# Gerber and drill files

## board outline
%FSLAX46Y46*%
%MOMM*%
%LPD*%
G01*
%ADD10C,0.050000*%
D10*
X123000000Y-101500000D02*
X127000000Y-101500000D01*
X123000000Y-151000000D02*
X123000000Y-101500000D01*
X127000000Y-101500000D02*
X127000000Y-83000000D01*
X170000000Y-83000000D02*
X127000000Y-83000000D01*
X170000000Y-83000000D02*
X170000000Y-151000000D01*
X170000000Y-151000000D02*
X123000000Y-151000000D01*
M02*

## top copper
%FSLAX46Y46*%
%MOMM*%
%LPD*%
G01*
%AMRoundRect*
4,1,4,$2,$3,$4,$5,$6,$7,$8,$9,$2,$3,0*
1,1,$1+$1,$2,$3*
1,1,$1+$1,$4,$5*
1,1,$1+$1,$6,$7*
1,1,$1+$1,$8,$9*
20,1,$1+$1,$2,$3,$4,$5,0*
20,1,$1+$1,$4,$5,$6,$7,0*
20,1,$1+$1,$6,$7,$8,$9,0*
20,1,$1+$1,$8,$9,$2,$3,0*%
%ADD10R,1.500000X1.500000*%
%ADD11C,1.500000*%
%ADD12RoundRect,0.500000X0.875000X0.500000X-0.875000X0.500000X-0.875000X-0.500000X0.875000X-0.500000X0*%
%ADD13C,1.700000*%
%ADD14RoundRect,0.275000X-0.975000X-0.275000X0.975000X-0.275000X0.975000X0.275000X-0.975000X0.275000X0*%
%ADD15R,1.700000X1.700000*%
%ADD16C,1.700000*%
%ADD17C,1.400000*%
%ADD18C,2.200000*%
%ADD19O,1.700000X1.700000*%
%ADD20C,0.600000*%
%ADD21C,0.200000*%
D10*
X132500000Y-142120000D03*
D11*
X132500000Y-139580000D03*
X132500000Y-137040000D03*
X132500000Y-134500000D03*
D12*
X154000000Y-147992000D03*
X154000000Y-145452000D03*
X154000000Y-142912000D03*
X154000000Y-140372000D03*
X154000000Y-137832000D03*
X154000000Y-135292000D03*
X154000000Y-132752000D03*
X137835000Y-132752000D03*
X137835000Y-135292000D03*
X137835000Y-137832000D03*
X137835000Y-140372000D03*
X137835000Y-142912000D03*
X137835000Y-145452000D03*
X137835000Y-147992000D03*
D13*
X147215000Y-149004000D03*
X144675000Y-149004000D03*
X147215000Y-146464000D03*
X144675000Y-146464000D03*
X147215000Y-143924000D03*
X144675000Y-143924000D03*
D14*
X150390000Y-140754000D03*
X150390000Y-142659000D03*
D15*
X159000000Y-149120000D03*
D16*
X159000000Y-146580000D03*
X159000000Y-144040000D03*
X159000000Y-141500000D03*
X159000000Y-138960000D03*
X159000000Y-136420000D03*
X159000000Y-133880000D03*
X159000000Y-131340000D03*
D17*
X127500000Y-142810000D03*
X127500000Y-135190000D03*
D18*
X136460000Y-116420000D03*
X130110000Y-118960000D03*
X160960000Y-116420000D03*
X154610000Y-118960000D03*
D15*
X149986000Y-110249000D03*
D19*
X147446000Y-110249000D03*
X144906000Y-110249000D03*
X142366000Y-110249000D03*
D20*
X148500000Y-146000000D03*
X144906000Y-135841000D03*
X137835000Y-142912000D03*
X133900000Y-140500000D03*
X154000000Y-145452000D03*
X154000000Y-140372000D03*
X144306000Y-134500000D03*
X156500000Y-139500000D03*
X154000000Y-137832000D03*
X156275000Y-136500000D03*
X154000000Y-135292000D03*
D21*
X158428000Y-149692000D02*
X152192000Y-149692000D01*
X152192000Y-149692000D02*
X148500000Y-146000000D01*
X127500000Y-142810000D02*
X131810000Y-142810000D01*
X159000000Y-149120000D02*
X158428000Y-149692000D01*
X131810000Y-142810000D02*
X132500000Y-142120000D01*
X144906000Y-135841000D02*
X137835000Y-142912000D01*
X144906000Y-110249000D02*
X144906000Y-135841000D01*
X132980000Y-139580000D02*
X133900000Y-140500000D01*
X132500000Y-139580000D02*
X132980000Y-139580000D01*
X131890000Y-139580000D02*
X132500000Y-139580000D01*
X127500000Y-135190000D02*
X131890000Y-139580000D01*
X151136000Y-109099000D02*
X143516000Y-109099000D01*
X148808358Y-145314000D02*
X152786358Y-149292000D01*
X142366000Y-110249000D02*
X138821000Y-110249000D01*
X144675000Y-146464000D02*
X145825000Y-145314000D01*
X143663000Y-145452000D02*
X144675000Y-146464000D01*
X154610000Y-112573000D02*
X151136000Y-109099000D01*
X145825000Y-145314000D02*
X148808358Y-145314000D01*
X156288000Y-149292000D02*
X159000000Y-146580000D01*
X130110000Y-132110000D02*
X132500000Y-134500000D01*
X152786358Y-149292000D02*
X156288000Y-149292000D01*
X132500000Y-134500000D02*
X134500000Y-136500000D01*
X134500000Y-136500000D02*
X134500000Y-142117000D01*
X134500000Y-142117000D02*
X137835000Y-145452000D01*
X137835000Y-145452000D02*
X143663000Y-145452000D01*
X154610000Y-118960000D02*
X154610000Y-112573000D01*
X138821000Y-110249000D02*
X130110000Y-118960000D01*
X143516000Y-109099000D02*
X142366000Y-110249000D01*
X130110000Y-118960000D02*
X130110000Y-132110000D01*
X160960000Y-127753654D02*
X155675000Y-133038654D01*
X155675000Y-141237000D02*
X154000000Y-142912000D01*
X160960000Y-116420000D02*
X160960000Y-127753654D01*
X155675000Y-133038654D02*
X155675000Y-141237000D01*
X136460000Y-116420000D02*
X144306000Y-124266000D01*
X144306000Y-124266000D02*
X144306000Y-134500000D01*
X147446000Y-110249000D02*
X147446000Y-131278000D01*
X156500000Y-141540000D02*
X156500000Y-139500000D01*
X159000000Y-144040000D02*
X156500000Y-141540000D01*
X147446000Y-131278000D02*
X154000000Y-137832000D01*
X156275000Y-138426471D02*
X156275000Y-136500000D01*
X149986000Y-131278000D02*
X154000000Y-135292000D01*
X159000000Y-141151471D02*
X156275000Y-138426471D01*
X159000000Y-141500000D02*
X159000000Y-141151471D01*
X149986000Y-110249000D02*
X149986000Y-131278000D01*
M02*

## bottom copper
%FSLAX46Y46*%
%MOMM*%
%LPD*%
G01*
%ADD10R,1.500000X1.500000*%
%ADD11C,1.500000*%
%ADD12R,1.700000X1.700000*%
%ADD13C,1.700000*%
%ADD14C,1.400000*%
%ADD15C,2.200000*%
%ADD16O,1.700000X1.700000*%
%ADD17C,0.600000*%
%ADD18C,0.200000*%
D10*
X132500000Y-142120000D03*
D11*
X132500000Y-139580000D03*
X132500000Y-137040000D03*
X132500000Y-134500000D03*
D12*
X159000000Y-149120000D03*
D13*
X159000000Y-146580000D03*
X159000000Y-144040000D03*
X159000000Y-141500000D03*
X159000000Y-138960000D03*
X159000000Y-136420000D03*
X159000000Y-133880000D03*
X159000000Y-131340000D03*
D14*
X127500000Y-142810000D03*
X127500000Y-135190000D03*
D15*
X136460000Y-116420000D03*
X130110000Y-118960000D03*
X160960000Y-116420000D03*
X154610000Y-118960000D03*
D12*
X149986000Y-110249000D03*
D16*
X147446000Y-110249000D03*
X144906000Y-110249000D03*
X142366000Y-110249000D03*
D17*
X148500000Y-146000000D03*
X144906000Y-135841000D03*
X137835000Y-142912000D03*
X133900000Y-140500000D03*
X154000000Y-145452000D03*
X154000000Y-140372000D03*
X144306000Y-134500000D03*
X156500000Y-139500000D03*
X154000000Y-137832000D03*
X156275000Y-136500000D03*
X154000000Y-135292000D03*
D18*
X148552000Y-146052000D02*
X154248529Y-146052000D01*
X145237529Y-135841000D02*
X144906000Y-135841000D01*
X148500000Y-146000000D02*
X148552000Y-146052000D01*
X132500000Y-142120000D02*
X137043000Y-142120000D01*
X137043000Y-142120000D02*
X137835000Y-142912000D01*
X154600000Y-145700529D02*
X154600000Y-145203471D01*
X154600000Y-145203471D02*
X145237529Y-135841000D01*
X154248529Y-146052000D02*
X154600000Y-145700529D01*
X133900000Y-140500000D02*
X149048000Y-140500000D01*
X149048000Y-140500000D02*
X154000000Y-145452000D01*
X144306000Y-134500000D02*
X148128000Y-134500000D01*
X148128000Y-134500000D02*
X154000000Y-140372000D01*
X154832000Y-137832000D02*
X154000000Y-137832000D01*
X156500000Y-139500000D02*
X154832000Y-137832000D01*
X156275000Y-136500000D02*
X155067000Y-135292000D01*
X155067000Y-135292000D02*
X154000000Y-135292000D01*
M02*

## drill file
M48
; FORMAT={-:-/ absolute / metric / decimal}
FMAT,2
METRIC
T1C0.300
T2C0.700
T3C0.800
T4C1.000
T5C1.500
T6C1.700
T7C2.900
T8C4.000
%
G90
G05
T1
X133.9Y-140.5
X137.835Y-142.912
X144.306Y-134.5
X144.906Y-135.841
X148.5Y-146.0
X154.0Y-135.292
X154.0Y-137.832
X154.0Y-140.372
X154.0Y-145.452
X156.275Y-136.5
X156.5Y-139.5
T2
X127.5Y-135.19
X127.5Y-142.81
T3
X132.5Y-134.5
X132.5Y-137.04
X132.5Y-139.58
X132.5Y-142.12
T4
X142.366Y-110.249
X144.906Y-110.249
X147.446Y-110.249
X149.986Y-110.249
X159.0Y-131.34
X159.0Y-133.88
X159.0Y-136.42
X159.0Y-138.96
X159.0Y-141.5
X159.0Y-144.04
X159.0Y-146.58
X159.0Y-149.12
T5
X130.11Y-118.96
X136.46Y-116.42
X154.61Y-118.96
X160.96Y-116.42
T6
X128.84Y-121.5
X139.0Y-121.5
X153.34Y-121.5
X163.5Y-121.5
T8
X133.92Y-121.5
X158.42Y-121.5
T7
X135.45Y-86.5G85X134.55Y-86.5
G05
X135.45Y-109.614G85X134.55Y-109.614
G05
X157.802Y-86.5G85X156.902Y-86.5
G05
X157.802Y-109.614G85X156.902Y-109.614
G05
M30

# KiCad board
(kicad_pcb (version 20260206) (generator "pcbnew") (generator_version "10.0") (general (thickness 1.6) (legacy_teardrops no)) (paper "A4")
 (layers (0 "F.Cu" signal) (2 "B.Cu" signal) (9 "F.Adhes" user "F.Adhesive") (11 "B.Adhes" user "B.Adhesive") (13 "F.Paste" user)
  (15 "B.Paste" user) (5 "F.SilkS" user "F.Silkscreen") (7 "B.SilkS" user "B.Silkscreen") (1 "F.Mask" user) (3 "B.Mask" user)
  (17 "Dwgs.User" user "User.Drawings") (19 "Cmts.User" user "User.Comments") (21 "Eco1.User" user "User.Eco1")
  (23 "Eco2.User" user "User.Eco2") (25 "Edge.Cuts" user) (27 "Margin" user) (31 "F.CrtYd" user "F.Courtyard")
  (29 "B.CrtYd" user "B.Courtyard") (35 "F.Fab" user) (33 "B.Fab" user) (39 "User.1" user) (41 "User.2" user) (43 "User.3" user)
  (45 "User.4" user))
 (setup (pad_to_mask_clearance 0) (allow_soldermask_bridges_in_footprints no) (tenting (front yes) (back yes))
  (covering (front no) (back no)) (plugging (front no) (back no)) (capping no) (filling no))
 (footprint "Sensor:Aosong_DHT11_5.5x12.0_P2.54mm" (layer "F.Cu") (at 132.5 142.12 180)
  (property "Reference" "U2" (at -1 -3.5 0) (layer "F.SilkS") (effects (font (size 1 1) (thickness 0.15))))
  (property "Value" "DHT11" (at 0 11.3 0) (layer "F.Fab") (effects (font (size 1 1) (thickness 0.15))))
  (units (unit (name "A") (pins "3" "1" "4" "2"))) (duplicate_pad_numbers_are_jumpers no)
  (pad "1" thru_hole rect (at 0 0 180) (size 1.5 1.5) (drill 0.8) (layers "*.Cu" "*.Mask") (remove_unused_layers no) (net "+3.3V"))
  (pad "2" thru_hole circle (at 0 2.54 180) (size 1.5 1.5) (drill 0.8) (layers "*.Cu" "*.Mask") (remove_unused_layers no)
   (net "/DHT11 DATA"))
  (pad "3" thru_hole circle (at 0 5.08 180) (size 1.5 1.5) (drill 0.8) (layers "*.Cu" "*.Mask") (remove_unused_layers no)
   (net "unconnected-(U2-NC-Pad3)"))
  (pad "4" thru_hole circle (at 0 7.62 180) (size 1.5 1.5) (drill 0.8) (layers "*.Cu" "*.Mask") (remove_unused_layers no) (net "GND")))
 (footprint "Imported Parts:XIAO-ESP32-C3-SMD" (layer "F.Cu") (at 154.835 129.872 180)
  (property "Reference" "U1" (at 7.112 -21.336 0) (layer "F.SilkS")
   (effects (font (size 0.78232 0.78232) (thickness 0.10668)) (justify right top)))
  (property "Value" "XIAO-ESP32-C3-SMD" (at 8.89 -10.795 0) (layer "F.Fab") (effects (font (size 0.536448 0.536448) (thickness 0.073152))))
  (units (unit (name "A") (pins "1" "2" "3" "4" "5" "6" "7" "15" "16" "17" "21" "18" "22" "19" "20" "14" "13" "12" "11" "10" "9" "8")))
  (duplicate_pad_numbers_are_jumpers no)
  (pad "1" smd roundrect (at 0.835 -18.12 180) (size 2.75 2) (layers "F.Cu" "F.Mask" "F.Paste") (roundrect_rratio 0.25)
   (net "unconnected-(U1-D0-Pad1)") (solder_mask_margin 0.0508) (thermal_bridge_angle 45))
  (pad "2" smd roundrect (at 0.835 -15.58 180) (size 2.75 2) (layers "F.Cu" "F.Mask" "F.Paste") (roundrect_rratio 0.25) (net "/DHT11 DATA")
   (solder_mask_margin 0.0508) (thermal_bridge_angle 45))
  (pad "3" smd roundrect (at 0.835 -13.04 180) (size 2.75 2) (layers "F.Cu" "F.Mask" "F.Paste") (roundrect_rratio 0.25) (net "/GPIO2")
   (solder_mask_margin 0.0508) (thermal_bridge_angle 45))
  (pad "4" smd roundrect (at 0.835 -10.5 180) (size 2.75 2) (layers "F.Cu" "F.Mask" "F.Paste") (roundrect_rratio 0.25) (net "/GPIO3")
   (solder_mask_margin 0.0508) (thermal_bridge_angle 45))
  (pad "5" smd roundrect (at 0.835 -7.96 180) (size 2.75 2) (layers "F.Cu" "F.Mask" "F.Paste") (roundrect_rratio 0.25) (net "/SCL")
   (solder_mask_margin 0.0508) (thermal_bridge_angle 45))
  (pad "6" smd roundrect (at 0.835 -5.42 180) (size 2.75 2) (layers "F.Cu" "F.Mask" "F.Paste") (roundrect_rratio 0.25) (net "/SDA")
   (solder_mask_margin 0.0508) (thermal_bridge_angle 45))
  (pad "7" smd roundrect (at 0.835 -2.88 180) (size 2.75 2) (layers "F.Cu" "F.Mask" "F.Paste") (roundrect_rratio 0.25)
   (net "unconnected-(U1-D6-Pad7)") (solder_mask_margin 0.0508) (thermal_bridge_angle 45))
  (pad "8" smd roundrect (at 17 -2.88 180) (size 2.75 2) (layers "F.Cu" "F.Mask" "F.Paste") (roundrect_rratio 0.25)
   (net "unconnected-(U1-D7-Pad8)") (solder_mask_margin 0.0508) (thermal_bridge_angle 45))
  (pad "9" smd roundrect (at 17 -5.42 180) (size 2.75 2) (layers "F.Cu" "F.Mask" "F.Paste") (roundrect_rratio 0.25)
   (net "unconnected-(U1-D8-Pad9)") (solder_mask_margin 0.0508) (thermal_bridge_angle 45))
  (pad "10" smd roundrect (at 17 -7.96 180) (size 2.75 2) (layers "F.Cu" "F.Mask" "F.Paste") (roundrect_rratio 0.25)
   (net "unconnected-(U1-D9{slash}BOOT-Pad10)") (solder_mask_margin 0.0508) (thermal_bridge_angle 45))
  (pad "11" smd roundrect (at 17 -10.5 180) (size 2.75 2) (layers "F.Cu" "F.Mask" "F.Paste") (roundrect_rratio 0.25)
   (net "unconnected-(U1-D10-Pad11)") (solder_mask_margin 0.0508) (thermal_bridge_angle 45))
  (pad "12" smd roundrect (at 17 -13.04 180) (size 2.75 2) (layers "F.Cu" "F.Mask" "F.Paste") (roundrect_rratio 0.25) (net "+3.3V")
   (solder_mask_margin 0.0508) (thermal_bridge_angle 45))
  (pad "13" smd roundrect (at 17 -15.58 180) (size 2.75 2) (layers "F.Cu" "F.Mask" "F.Paste") (roundrect_rratio 0.25) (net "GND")
   (solder_mask_margin 0.0508) (thermal_bridge_angle 45))
  (pad "14" smd roundrect (at 17 -18.12 180) (size 2.75 2) (layers "F.Cu" "F.Mask" "F.Paste") (roundrect_rratio 0.25) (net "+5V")
   (solder_mask_margin 0.0508) (thermal_bridge_angle 45))
  (pad "15" smd circle (at 7.62 -19.132 180) (size 1.7 1.7) (layers "F.Cu" "F.Mask" "F.Paste") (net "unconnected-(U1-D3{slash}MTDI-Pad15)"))
  (pad "16" smd circle (at 10.16 -19.132 180) (size 1.7 1.7) (layers "F.Cu" "F.Mask" "F.Paste") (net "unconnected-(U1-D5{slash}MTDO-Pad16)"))
  (pad "17" smd circle (at 7.62 -16.592 180) (size 1.7 1.7) (layers "F.Cu" "F.Mask" "F.Paste") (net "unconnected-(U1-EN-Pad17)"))
  (pad "18" smd circle (at 10.16 -16.592 180) (size 1.7 1.7) (layers "F.Cu" "F.Mask" "F.Paste") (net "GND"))
  (pad "19" smd circle (at 7.62 -14.052 180) (size 1.7 1.7) (layers "F.Cu" "F.Mask" "F.Paste") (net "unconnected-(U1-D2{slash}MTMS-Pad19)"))
  (pad "20" smd circle (at 10.16 -14.052 180) (size 1.7 1.7) (layers "F.Cu" "F.Mask" "F.Paste") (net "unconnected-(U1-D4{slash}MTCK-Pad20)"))
  (pad "21" smd roundrect (at 4.445 -10.882) (size 2.5 1.1) (layers "F.Cu" "F.Mask" "F.Paste") (roundrect_rratio 0.25)
   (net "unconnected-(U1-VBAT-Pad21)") (thermal_bridge_angle 45))
  (pad "22" smd roundrect (at 4.445 -12.787) (size 2.5 1.1) (layers "F.Cu" "F.Mask" "F.Paste") (roundrect_rratio 0.25)
   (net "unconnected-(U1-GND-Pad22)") (thermal_bridge_angle 45)))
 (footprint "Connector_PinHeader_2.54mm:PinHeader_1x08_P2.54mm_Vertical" (layer "F.Cu") (at 159 149.12 180)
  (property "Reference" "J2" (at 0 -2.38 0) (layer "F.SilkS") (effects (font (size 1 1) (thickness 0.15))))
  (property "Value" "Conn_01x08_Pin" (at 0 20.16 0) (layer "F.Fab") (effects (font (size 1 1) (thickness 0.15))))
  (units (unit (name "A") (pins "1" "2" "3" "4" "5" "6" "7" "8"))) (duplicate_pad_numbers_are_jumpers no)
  (pad "1" thru_hole rect (at 0 0 180) (size 1.7 1.7) (drill 1) (layers "*.Cu" "*.Mask") (remove_unused_layers no) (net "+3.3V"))
  (pad "2" thru_hole circle (at 0 2.54 180) (size 1.7 1.7) (drill 1) (layers "*.Cu" "*.Mask") (remove_unused_layers no) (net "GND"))
  (pad "3" thru_hole circle (at 0 5.08 180) (size 1.7 1.7) (drill 1) (layers "*.Cu" "*.Mask") (remove_unused_layers no) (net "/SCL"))
  (pad "4" thru_hole circle (at 0 7.62 180) (size 1.7 1.7) (drill 1) (layers "*.Cu" "*.Mask") (remove_unused_layers no) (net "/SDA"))
  (pad "5" thru_hole circle (at 0 10.16 180) (size 1.7 1.7) (drill 1) (layers "*.Cu" "*.Mask") (remove_unused_layers no)
   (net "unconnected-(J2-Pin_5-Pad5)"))
  (pad "6" thru_hole circle (at 0 12.7 180) (size 1.7 1.7) (drill 1) (layers "*.Cu" "*.Mask") (remove_unused_layers no)
   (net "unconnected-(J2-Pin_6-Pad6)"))
  (pad "7" thru_hole circle (at 0 15.24 180) (size 1.7 1.7) (drill 1) (layers "*.Cu" "*.Mask") (remove_unused_layers no)
   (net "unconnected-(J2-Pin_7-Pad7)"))
  (pad "8" thru_hole circle (at 0 17.78 180) (size 1.7 1.7) (drill 1) (layers "*.Cu" "*.Mask") (remove_unused_layers no)
   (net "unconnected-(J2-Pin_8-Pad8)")))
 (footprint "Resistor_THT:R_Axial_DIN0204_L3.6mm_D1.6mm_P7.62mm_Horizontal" (layer "F.Cu") (at 127.5 142.81 90)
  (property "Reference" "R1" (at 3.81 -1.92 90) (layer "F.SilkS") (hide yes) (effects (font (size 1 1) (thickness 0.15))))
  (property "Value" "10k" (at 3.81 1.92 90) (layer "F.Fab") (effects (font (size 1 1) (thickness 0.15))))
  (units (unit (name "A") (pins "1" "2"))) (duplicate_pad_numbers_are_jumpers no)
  (pad "1" thru_hole circle (at 0 0 90) (size 1.4 1.4) (drill 0.7) (layers "*.Cu" "*.Mask") (remove_unused_layers no) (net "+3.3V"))
  (pad "2" thru_hole circle (at 7.62 0 90) (size 1.4 1.4) (drill 0.7) (layers "*.Cu" "*.Mask") (remove_unused_layers no) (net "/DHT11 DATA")))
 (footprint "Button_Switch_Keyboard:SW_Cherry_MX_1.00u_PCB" (layer "F.Cu") (at 136.46 116.42)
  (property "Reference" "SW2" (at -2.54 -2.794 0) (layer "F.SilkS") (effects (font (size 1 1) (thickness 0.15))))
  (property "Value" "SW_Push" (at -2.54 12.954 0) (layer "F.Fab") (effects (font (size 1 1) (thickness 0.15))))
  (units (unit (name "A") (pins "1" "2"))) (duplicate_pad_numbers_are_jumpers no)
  (pad "" np_thru_hole circle (at -7.62 5.08) (size 1.7 1.7) (drill 1.7) (layers "*.Cu" "*.Mask"))
  (pad "" np_thru_hole circle (at -2.54 5.08) (size 4 4) (drill 4) (layers "*.Cu" "*.Mask"))
  (pad "" np_thru_hole circle (at 2.54 5.08) (size 1.7 1.7) (drill 1.7) (layers "*.Cu" "*.Mask"))
  (pad "1" thru_hole circle (at 0 0) (size 2.2 2.2) (drill 1.5) (layers "*.Cu" "*.Mask") (remove_unused_layers no) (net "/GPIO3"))
  (pad "2" thru_hole circle (at -6.35 2.54) (size 2.2 2.2) (drill 1.5) (layers "*.Cu" "*.Mask") (remove_unused_layers no) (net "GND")))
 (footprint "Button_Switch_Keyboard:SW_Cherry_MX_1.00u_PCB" (layer "F.Cu") (at 160.96 116.42)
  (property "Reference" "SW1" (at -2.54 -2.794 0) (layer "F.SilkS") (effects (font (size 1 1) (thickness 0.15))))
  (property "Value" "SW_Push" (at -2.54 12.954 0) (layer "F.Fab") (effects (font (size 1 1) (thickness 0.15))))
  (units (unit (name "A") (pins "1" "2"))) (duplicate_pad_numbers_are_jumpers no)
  (pad "" np_thru_hole circle (at -7.62 5.08) (size 1.7 1.7) (drill 1.7) (layers "*.Cu" "*.Mask"))
  (pad "" np_thru_hole circle (at -2.54 5.08) (size 4 4) (drill 4) (layers "*.Cu" "*.Mask"))
  (pad "" np_thru_hole circle (at 2.54 5.08) (size 1.7 1.7) (drill 1.7) (layers "*.Cu" "*.Mask"))
  (pad "1" thru_hole circle (at 0 0) (size 2.2 2.2) (drill 1.5) (layers "*.Cu" "*.Mask") (remove_unused_layers no) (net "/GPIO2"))
  (pad "2" thru_hole circle (at -6.35 2.54) (size 2.2 2.2) (drill 1.5) (layers "*.Cu" "*.Mask") (remove_unused_layers no) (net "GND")))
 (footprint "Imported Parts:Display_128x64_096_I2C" (layer "F.Cu") (at 146.176 110.249 180)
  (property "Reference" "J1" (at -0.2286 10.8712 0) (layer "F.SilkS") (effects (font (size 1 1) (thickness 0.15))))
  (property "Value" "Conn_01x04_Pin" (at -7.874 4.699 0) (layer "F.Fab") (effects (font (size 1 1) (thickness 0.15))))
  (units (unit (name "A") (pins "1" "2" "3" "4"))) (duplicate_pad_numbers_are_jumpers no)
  (pad "" np_thru_hole oval (at -11.176 0.635 180) (size 3.8 2.9) (drill oval 3.8 2.9) (layers "*.Cu" "*.Mask"))
  (pad "" np_thru_hole oval (at -11.176 23.749 180) (size 3.8 2.9) (drill oval 3.8 2.9) (layers "*.Cu" "*.Mask"))
  (pad "" np_thru_hole oval (at 11.176 0.635 180) (size 3.8 2.9) (drill oval 3.8 2.9) (layers "*.Cu" "*.Mask"))
  (pad "" np_thru_hole oval (at 11.176 23.749 180) (size 3.8 2.9) (drill oval 3.8 2.9) (layers "*.Cu" "*.Mask"))
  (pad "1" thru_hole rect (at -3.81 0 270) (size 1.7 1.7) (drill 1) (layers "*.Cu" "*.Mask") (remove_unused_layers no) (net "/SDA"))
  (pad "2" thru_hole oval (at -1.27 0 270) (size 1.7 1.7) (drill 1) (layers "*.Cu" "*.Mask") (remove_unused_layers no) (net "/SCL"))
  (pad "3" thru_hole oval (at 1.27 0 270) (size 1.7 1.7) (drill 1) (layers "*.Cu" "*.Mask") (remove_unused_layers no) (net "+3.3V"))
  (pad "4" thru_hole oval (at 3.81 0 270) (size 1.7 1.7) (drill 1) (layers "*.Cu" "*.Mask") (remove_unused_layers no) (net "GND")))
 (gr_line (start 123 101.5) (end 127 101.5) (stroke (width 0.05) (type default)) (layer "Edge.Cuts"))
 (gr_line (start 123 151) (end 123 101.5) (stroke (width 0.05) (type default)) (layer "Edge.Cuts"))
 (gr_line (start 127 101.5) (end 127 83) (stroke (width 0.05) (type default)) (layer "Edge.Cuts"))
 (gr_line (start 170 83) (end 127 83) (stroke (width 0.05) (type default)) (layer "Edge.Cuts"))
 (gr_line (start 170 83) (end 170 151) (stroke (width 0.05) (type default)) (layer "Edge.Cuts"))
 (gr_line (start 170 151) (end 123 151) (stroke (width 0.05) (type default)) (layer "Edge.Cuts"))
 (segment (start 158.428 149.692) (end 152.192 149.692) (width 0.2) (layer "F.Cu") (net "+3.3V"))
 (segment (start 152.192 149.692) (end 148.5 146) (width 0.2) (layer "F.Cu") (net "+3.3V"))
 (segment (start 127.5 142.81) (end 131.81 142.81) (width 0.2) (layer "F.Cu") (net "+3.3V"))
 (segment (start 159 149.12) (end 158.428 149.692) (width 0.2) (layer "F.Cu") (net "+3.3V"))
 (segment (start 131.81 142.81) (end 132.5 142.12) (width 0.2) (layer "F.Cu") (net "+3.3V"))
 (segment (start 144.906 135.841) (end 137.835 142.912) (width 0.2) (layer "F.Cu") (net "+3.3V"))
 (segment (start 144.906 110.249) (end 144.906 135.841) (width 0.2) (layer "F.Cu") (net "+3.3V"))
 (via (at 148.5 146) (size 0.6) (drill 0.3) (layers "F.Cu" "B.Cu") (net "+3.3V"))
 (via (at 144.906 135.841) (size 0.6) (drill 0.3) (layers "F.Cu" "B.Cu") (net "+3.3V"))
 (via (at 137.835 142.912) (size 0.6) (drill 0.3) (layers "F.Cu" "B.Cu") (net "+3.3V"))
 (segment (start 148.552 146.052) (end 154.248529 146.052) (width 0.2) (layer "B.Cu") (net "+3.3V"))
 (segment (start 145.237529 135.841) (end 144.906 135.841) (width 0.2) (layer "B.Cu") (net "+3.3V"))
 (segment (start 148.5 146) (end 148.552 146.052) (width 0.2) (layer "B.Cu") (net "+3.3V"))
 (segment (start 132.5 142.12) (end 137.043 142.12) (width 0.2) (layer "B.Cu") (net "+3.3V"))
 (segment (start 137.043 142.12) (end 137.835 142.912) (width 0.2) (layer "B.Cu") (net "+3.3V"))
 (segment (start 154.6 145.700529) (end 154.6 145.203471) (width 0.2) (layer "B.Cu") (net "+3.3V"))
 (segment (start 154.6 145.203471) (end 145.237529 135.841) (width 0.2) (layer "B.Cu") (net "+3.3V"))
 (segment (start 154.248529 146.052) (end 154.6 145.700529) (width 0.2) (layer "B.Cu") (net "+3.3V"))
 (segment (start 132.98 139.58) (end 133.9 140.5) (width 0.2) (layer "F.Cu") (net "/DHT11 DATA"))
 (segment (start 132.5 139.58) (end 132.98 139.58) (width 0.2) (layer "F.Cu") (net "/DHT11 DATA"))
 (segment (start 131.89 139.58) (end 132.5 139.58) (width 0.2) (layer "F.Cu") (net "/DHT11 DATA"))
 (segment (start 127.5 135.19) (end 131.89 139.58) (width 0.2) (layer "F.Cu") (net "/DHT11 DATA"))
 (via (at 133.9 140.5) (size 0.6) (drill 0.3) (layers "F.Cu" "B.Cu") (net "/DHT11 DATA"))
 (via (at 154 145.452) (size 0.6) (drill 0.3) (layers "F.Cu" "B.Cu") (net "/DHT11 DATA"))
 (segment (start 133.9 140.5) (end 149.048 140.5) (width 0.2) (layer "B.Cu") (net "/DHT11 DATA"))
 (segment (start 149.048 140.5) (end 154 145.452) (width 0.2) (layer "B.Cu") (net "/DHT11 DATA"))
 (segment (start 151.136 109.099) (end 143.516 109.099) (width 0.2) (layer "F.Cu") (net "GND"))
 (segment (start 148.808358 145.314) (end 152.786358 149.292) (width 0.2) (layer "F.Cu") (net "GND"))
 (segment (start 142.366 110.249) (end 138.821 110.249) (width 0.2) (layer "F.Cu") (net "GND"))
 (segment (start 144.675 146.464) (end 145.825 145.314) (width 0.2) (layer "F.Cu") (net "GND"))
 (segment (start 143.663 145.452) (end 144.675 146.464) (width 0.2) (layer "F.Cu") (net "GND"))
 (segment (start 154.61 112.573) (end 151.136 109.099) (width 0.2) (layer "F.Cu") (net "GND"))
 (segment (start 145.825 145.314) (end 148.808358 145.314) (width 0.2) (layer "F.Cu") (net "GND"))
 (segment (start 156.288 149.292) (end 159 146.58) (width 0.2) (layer "F.Cu") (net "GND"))
 (segment (start 130.11 132.11) (end 132.5 134.5) (width 0.2) (layer "F.Cu") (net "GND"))
 (segment (start 152.786358 149.292) (end 156.288 149.292) (width 0.2) (layer "F.Cu") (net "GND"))
 (segment (start 132.5 134.5) (end 134.5 136.5) (width 0.2) (layer "F.Cu") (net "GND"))
 (segment (start 134.5 136.5) (end 134.5 142.117) (width 0.2) (layer "F.Cu") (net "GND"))
 (segment (start 134.5 142.117) (end 137.835 145.452) (width 0.2) (layer "F.Cu") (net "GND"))
 (segment (start 137.835 145.452) (end 143.663 145.452) (width 0.2) (layer "F.Cu") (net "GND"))
 (segment (start 154.61 118.96) (end 154.61 112.573) (width 0.2) (layer "F.Cu") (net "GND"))
 (segment (start 138.821 110.249) (end 130.11 118.96) (width 0.2) (layer "F.Cu") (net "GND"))
 (segment (start 143.516 109.099) (end 142.366 110.249) (width 0.2) (layer "F.Cu") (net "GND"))
 (segment (start 130.11 118.96) (end 130.11 132.11) (width 0.2) (layer "F.Cu") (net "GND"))
 (segment (start 160.96 127.753654) (end 155.675 133.038654) (width 0.2) (layer "F.Cu") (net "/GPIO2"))
 (segment (start 155.675 141.237) (end 154 142.912) (width 0.2) (layer "F.Cu") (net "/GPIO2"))
 (segment (start 160.96 116.42) (end 160.96 127.753654) (width 0.2) (layer "F.Cu") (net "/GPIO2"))
 (segment (start 155.675 133.038654) (end 155.675 141.237) (width 0.2) (layer "F.Cu") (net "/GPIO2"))
 (segment (start 136.46 116.42) (end 144.306 124.266) (width 0.2) (layer "F.Cu") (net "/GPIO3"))
 (segment (start 144.306 124.266) (end 144.306 134.5) (width 0.2) (layer "F.Cu") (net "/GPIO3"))
 (via (at 154 140.372) (size 0.6) (drill 0.3) (layers "F.Cu" "B.Cu") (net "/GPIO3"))
 (via (at 144.306 134.5) (size 0.6) (drill 0.3) (layers "F.Cu" "B.Cu") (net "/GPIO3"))
 (segment (start 144.306 134.5) (end 148.128 134.5) (width 0.2) (layer "B.Cu") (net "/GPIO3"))
 (segment (start 148.128 134.5) (end 154 140.372) (width 0.2) (layer "B.Cu") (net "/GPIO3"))
 (segment (start 147.446 110.249) (end 147.446 131.278) (width 0.2) (layer "F.Cu") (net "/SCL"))
 (segment (start 156.5 141.54) (end 156.5 139.5) (width 0.2) (layer "F.Cu") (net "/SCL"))
 (segment (start 159 144.04) (end 156.5 141.54) (width 0.2) (layer "F.Cu") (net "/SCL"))
 (segment (start 147.446 131.278) (end 154 137.832) (width 0.2) (layer "F.Cu") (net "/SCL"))
 (via (at 156.5 139.5) (size 0.6) (drill 0.3) (layers "F.Cu" "B.Cu") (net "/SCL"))
 (via (at 154 137.832) (size 0.6) (drill 0.3) (layers "F.Cu" "B.Cu") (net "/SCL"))
 (segment (start 154.832 137.832) (end 154 137.832) (width 0.2) (layer "B.Cu") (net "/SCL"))
 (segment (start 156.5 139.5) (end 154.832 137.832) (width 0.2) (layer "B.Cu") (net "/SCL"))
 (segment (start 156.275 138.426471) (end 156.275 136.5) (width 0.2) (layer "F.Cu") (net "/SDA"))
 (segment (start 149.986 131.278) (end 154 135.292) (width 0.2) (layer "F.Cu") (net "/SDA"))
 (segment (start 159 141.151471) (end 156.275 138.426471) (width 0.2) (layer "F.Cu") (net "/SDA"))
 (segment (start 159 141.5) (end 159 141.151471) (width 0.2) (layer "F.Cu") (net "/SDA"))
 (segment (start 149.986 110.249) (end 149.986 131.278) (width 0.2) (layer "F.Cu") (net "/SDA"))
 (via (at 156.275 136.5) (size 0.6) (drill 0.3) (layers "F.Cu" "B.Cu") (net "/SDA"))
 (via (at 154 135.292) (size 0.6) (drill 0.3) (layers "F.Cu" "B.Cu") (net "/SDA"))
 (segment (start 156.275 136.5) (end 155.067 135.292) (width 0.2) (layer "B.Cu") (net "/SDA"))
 (segment (start 155.067 135.292) (end 154 135.292) (width 0.2) (layer "B.Cu") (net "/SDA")))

